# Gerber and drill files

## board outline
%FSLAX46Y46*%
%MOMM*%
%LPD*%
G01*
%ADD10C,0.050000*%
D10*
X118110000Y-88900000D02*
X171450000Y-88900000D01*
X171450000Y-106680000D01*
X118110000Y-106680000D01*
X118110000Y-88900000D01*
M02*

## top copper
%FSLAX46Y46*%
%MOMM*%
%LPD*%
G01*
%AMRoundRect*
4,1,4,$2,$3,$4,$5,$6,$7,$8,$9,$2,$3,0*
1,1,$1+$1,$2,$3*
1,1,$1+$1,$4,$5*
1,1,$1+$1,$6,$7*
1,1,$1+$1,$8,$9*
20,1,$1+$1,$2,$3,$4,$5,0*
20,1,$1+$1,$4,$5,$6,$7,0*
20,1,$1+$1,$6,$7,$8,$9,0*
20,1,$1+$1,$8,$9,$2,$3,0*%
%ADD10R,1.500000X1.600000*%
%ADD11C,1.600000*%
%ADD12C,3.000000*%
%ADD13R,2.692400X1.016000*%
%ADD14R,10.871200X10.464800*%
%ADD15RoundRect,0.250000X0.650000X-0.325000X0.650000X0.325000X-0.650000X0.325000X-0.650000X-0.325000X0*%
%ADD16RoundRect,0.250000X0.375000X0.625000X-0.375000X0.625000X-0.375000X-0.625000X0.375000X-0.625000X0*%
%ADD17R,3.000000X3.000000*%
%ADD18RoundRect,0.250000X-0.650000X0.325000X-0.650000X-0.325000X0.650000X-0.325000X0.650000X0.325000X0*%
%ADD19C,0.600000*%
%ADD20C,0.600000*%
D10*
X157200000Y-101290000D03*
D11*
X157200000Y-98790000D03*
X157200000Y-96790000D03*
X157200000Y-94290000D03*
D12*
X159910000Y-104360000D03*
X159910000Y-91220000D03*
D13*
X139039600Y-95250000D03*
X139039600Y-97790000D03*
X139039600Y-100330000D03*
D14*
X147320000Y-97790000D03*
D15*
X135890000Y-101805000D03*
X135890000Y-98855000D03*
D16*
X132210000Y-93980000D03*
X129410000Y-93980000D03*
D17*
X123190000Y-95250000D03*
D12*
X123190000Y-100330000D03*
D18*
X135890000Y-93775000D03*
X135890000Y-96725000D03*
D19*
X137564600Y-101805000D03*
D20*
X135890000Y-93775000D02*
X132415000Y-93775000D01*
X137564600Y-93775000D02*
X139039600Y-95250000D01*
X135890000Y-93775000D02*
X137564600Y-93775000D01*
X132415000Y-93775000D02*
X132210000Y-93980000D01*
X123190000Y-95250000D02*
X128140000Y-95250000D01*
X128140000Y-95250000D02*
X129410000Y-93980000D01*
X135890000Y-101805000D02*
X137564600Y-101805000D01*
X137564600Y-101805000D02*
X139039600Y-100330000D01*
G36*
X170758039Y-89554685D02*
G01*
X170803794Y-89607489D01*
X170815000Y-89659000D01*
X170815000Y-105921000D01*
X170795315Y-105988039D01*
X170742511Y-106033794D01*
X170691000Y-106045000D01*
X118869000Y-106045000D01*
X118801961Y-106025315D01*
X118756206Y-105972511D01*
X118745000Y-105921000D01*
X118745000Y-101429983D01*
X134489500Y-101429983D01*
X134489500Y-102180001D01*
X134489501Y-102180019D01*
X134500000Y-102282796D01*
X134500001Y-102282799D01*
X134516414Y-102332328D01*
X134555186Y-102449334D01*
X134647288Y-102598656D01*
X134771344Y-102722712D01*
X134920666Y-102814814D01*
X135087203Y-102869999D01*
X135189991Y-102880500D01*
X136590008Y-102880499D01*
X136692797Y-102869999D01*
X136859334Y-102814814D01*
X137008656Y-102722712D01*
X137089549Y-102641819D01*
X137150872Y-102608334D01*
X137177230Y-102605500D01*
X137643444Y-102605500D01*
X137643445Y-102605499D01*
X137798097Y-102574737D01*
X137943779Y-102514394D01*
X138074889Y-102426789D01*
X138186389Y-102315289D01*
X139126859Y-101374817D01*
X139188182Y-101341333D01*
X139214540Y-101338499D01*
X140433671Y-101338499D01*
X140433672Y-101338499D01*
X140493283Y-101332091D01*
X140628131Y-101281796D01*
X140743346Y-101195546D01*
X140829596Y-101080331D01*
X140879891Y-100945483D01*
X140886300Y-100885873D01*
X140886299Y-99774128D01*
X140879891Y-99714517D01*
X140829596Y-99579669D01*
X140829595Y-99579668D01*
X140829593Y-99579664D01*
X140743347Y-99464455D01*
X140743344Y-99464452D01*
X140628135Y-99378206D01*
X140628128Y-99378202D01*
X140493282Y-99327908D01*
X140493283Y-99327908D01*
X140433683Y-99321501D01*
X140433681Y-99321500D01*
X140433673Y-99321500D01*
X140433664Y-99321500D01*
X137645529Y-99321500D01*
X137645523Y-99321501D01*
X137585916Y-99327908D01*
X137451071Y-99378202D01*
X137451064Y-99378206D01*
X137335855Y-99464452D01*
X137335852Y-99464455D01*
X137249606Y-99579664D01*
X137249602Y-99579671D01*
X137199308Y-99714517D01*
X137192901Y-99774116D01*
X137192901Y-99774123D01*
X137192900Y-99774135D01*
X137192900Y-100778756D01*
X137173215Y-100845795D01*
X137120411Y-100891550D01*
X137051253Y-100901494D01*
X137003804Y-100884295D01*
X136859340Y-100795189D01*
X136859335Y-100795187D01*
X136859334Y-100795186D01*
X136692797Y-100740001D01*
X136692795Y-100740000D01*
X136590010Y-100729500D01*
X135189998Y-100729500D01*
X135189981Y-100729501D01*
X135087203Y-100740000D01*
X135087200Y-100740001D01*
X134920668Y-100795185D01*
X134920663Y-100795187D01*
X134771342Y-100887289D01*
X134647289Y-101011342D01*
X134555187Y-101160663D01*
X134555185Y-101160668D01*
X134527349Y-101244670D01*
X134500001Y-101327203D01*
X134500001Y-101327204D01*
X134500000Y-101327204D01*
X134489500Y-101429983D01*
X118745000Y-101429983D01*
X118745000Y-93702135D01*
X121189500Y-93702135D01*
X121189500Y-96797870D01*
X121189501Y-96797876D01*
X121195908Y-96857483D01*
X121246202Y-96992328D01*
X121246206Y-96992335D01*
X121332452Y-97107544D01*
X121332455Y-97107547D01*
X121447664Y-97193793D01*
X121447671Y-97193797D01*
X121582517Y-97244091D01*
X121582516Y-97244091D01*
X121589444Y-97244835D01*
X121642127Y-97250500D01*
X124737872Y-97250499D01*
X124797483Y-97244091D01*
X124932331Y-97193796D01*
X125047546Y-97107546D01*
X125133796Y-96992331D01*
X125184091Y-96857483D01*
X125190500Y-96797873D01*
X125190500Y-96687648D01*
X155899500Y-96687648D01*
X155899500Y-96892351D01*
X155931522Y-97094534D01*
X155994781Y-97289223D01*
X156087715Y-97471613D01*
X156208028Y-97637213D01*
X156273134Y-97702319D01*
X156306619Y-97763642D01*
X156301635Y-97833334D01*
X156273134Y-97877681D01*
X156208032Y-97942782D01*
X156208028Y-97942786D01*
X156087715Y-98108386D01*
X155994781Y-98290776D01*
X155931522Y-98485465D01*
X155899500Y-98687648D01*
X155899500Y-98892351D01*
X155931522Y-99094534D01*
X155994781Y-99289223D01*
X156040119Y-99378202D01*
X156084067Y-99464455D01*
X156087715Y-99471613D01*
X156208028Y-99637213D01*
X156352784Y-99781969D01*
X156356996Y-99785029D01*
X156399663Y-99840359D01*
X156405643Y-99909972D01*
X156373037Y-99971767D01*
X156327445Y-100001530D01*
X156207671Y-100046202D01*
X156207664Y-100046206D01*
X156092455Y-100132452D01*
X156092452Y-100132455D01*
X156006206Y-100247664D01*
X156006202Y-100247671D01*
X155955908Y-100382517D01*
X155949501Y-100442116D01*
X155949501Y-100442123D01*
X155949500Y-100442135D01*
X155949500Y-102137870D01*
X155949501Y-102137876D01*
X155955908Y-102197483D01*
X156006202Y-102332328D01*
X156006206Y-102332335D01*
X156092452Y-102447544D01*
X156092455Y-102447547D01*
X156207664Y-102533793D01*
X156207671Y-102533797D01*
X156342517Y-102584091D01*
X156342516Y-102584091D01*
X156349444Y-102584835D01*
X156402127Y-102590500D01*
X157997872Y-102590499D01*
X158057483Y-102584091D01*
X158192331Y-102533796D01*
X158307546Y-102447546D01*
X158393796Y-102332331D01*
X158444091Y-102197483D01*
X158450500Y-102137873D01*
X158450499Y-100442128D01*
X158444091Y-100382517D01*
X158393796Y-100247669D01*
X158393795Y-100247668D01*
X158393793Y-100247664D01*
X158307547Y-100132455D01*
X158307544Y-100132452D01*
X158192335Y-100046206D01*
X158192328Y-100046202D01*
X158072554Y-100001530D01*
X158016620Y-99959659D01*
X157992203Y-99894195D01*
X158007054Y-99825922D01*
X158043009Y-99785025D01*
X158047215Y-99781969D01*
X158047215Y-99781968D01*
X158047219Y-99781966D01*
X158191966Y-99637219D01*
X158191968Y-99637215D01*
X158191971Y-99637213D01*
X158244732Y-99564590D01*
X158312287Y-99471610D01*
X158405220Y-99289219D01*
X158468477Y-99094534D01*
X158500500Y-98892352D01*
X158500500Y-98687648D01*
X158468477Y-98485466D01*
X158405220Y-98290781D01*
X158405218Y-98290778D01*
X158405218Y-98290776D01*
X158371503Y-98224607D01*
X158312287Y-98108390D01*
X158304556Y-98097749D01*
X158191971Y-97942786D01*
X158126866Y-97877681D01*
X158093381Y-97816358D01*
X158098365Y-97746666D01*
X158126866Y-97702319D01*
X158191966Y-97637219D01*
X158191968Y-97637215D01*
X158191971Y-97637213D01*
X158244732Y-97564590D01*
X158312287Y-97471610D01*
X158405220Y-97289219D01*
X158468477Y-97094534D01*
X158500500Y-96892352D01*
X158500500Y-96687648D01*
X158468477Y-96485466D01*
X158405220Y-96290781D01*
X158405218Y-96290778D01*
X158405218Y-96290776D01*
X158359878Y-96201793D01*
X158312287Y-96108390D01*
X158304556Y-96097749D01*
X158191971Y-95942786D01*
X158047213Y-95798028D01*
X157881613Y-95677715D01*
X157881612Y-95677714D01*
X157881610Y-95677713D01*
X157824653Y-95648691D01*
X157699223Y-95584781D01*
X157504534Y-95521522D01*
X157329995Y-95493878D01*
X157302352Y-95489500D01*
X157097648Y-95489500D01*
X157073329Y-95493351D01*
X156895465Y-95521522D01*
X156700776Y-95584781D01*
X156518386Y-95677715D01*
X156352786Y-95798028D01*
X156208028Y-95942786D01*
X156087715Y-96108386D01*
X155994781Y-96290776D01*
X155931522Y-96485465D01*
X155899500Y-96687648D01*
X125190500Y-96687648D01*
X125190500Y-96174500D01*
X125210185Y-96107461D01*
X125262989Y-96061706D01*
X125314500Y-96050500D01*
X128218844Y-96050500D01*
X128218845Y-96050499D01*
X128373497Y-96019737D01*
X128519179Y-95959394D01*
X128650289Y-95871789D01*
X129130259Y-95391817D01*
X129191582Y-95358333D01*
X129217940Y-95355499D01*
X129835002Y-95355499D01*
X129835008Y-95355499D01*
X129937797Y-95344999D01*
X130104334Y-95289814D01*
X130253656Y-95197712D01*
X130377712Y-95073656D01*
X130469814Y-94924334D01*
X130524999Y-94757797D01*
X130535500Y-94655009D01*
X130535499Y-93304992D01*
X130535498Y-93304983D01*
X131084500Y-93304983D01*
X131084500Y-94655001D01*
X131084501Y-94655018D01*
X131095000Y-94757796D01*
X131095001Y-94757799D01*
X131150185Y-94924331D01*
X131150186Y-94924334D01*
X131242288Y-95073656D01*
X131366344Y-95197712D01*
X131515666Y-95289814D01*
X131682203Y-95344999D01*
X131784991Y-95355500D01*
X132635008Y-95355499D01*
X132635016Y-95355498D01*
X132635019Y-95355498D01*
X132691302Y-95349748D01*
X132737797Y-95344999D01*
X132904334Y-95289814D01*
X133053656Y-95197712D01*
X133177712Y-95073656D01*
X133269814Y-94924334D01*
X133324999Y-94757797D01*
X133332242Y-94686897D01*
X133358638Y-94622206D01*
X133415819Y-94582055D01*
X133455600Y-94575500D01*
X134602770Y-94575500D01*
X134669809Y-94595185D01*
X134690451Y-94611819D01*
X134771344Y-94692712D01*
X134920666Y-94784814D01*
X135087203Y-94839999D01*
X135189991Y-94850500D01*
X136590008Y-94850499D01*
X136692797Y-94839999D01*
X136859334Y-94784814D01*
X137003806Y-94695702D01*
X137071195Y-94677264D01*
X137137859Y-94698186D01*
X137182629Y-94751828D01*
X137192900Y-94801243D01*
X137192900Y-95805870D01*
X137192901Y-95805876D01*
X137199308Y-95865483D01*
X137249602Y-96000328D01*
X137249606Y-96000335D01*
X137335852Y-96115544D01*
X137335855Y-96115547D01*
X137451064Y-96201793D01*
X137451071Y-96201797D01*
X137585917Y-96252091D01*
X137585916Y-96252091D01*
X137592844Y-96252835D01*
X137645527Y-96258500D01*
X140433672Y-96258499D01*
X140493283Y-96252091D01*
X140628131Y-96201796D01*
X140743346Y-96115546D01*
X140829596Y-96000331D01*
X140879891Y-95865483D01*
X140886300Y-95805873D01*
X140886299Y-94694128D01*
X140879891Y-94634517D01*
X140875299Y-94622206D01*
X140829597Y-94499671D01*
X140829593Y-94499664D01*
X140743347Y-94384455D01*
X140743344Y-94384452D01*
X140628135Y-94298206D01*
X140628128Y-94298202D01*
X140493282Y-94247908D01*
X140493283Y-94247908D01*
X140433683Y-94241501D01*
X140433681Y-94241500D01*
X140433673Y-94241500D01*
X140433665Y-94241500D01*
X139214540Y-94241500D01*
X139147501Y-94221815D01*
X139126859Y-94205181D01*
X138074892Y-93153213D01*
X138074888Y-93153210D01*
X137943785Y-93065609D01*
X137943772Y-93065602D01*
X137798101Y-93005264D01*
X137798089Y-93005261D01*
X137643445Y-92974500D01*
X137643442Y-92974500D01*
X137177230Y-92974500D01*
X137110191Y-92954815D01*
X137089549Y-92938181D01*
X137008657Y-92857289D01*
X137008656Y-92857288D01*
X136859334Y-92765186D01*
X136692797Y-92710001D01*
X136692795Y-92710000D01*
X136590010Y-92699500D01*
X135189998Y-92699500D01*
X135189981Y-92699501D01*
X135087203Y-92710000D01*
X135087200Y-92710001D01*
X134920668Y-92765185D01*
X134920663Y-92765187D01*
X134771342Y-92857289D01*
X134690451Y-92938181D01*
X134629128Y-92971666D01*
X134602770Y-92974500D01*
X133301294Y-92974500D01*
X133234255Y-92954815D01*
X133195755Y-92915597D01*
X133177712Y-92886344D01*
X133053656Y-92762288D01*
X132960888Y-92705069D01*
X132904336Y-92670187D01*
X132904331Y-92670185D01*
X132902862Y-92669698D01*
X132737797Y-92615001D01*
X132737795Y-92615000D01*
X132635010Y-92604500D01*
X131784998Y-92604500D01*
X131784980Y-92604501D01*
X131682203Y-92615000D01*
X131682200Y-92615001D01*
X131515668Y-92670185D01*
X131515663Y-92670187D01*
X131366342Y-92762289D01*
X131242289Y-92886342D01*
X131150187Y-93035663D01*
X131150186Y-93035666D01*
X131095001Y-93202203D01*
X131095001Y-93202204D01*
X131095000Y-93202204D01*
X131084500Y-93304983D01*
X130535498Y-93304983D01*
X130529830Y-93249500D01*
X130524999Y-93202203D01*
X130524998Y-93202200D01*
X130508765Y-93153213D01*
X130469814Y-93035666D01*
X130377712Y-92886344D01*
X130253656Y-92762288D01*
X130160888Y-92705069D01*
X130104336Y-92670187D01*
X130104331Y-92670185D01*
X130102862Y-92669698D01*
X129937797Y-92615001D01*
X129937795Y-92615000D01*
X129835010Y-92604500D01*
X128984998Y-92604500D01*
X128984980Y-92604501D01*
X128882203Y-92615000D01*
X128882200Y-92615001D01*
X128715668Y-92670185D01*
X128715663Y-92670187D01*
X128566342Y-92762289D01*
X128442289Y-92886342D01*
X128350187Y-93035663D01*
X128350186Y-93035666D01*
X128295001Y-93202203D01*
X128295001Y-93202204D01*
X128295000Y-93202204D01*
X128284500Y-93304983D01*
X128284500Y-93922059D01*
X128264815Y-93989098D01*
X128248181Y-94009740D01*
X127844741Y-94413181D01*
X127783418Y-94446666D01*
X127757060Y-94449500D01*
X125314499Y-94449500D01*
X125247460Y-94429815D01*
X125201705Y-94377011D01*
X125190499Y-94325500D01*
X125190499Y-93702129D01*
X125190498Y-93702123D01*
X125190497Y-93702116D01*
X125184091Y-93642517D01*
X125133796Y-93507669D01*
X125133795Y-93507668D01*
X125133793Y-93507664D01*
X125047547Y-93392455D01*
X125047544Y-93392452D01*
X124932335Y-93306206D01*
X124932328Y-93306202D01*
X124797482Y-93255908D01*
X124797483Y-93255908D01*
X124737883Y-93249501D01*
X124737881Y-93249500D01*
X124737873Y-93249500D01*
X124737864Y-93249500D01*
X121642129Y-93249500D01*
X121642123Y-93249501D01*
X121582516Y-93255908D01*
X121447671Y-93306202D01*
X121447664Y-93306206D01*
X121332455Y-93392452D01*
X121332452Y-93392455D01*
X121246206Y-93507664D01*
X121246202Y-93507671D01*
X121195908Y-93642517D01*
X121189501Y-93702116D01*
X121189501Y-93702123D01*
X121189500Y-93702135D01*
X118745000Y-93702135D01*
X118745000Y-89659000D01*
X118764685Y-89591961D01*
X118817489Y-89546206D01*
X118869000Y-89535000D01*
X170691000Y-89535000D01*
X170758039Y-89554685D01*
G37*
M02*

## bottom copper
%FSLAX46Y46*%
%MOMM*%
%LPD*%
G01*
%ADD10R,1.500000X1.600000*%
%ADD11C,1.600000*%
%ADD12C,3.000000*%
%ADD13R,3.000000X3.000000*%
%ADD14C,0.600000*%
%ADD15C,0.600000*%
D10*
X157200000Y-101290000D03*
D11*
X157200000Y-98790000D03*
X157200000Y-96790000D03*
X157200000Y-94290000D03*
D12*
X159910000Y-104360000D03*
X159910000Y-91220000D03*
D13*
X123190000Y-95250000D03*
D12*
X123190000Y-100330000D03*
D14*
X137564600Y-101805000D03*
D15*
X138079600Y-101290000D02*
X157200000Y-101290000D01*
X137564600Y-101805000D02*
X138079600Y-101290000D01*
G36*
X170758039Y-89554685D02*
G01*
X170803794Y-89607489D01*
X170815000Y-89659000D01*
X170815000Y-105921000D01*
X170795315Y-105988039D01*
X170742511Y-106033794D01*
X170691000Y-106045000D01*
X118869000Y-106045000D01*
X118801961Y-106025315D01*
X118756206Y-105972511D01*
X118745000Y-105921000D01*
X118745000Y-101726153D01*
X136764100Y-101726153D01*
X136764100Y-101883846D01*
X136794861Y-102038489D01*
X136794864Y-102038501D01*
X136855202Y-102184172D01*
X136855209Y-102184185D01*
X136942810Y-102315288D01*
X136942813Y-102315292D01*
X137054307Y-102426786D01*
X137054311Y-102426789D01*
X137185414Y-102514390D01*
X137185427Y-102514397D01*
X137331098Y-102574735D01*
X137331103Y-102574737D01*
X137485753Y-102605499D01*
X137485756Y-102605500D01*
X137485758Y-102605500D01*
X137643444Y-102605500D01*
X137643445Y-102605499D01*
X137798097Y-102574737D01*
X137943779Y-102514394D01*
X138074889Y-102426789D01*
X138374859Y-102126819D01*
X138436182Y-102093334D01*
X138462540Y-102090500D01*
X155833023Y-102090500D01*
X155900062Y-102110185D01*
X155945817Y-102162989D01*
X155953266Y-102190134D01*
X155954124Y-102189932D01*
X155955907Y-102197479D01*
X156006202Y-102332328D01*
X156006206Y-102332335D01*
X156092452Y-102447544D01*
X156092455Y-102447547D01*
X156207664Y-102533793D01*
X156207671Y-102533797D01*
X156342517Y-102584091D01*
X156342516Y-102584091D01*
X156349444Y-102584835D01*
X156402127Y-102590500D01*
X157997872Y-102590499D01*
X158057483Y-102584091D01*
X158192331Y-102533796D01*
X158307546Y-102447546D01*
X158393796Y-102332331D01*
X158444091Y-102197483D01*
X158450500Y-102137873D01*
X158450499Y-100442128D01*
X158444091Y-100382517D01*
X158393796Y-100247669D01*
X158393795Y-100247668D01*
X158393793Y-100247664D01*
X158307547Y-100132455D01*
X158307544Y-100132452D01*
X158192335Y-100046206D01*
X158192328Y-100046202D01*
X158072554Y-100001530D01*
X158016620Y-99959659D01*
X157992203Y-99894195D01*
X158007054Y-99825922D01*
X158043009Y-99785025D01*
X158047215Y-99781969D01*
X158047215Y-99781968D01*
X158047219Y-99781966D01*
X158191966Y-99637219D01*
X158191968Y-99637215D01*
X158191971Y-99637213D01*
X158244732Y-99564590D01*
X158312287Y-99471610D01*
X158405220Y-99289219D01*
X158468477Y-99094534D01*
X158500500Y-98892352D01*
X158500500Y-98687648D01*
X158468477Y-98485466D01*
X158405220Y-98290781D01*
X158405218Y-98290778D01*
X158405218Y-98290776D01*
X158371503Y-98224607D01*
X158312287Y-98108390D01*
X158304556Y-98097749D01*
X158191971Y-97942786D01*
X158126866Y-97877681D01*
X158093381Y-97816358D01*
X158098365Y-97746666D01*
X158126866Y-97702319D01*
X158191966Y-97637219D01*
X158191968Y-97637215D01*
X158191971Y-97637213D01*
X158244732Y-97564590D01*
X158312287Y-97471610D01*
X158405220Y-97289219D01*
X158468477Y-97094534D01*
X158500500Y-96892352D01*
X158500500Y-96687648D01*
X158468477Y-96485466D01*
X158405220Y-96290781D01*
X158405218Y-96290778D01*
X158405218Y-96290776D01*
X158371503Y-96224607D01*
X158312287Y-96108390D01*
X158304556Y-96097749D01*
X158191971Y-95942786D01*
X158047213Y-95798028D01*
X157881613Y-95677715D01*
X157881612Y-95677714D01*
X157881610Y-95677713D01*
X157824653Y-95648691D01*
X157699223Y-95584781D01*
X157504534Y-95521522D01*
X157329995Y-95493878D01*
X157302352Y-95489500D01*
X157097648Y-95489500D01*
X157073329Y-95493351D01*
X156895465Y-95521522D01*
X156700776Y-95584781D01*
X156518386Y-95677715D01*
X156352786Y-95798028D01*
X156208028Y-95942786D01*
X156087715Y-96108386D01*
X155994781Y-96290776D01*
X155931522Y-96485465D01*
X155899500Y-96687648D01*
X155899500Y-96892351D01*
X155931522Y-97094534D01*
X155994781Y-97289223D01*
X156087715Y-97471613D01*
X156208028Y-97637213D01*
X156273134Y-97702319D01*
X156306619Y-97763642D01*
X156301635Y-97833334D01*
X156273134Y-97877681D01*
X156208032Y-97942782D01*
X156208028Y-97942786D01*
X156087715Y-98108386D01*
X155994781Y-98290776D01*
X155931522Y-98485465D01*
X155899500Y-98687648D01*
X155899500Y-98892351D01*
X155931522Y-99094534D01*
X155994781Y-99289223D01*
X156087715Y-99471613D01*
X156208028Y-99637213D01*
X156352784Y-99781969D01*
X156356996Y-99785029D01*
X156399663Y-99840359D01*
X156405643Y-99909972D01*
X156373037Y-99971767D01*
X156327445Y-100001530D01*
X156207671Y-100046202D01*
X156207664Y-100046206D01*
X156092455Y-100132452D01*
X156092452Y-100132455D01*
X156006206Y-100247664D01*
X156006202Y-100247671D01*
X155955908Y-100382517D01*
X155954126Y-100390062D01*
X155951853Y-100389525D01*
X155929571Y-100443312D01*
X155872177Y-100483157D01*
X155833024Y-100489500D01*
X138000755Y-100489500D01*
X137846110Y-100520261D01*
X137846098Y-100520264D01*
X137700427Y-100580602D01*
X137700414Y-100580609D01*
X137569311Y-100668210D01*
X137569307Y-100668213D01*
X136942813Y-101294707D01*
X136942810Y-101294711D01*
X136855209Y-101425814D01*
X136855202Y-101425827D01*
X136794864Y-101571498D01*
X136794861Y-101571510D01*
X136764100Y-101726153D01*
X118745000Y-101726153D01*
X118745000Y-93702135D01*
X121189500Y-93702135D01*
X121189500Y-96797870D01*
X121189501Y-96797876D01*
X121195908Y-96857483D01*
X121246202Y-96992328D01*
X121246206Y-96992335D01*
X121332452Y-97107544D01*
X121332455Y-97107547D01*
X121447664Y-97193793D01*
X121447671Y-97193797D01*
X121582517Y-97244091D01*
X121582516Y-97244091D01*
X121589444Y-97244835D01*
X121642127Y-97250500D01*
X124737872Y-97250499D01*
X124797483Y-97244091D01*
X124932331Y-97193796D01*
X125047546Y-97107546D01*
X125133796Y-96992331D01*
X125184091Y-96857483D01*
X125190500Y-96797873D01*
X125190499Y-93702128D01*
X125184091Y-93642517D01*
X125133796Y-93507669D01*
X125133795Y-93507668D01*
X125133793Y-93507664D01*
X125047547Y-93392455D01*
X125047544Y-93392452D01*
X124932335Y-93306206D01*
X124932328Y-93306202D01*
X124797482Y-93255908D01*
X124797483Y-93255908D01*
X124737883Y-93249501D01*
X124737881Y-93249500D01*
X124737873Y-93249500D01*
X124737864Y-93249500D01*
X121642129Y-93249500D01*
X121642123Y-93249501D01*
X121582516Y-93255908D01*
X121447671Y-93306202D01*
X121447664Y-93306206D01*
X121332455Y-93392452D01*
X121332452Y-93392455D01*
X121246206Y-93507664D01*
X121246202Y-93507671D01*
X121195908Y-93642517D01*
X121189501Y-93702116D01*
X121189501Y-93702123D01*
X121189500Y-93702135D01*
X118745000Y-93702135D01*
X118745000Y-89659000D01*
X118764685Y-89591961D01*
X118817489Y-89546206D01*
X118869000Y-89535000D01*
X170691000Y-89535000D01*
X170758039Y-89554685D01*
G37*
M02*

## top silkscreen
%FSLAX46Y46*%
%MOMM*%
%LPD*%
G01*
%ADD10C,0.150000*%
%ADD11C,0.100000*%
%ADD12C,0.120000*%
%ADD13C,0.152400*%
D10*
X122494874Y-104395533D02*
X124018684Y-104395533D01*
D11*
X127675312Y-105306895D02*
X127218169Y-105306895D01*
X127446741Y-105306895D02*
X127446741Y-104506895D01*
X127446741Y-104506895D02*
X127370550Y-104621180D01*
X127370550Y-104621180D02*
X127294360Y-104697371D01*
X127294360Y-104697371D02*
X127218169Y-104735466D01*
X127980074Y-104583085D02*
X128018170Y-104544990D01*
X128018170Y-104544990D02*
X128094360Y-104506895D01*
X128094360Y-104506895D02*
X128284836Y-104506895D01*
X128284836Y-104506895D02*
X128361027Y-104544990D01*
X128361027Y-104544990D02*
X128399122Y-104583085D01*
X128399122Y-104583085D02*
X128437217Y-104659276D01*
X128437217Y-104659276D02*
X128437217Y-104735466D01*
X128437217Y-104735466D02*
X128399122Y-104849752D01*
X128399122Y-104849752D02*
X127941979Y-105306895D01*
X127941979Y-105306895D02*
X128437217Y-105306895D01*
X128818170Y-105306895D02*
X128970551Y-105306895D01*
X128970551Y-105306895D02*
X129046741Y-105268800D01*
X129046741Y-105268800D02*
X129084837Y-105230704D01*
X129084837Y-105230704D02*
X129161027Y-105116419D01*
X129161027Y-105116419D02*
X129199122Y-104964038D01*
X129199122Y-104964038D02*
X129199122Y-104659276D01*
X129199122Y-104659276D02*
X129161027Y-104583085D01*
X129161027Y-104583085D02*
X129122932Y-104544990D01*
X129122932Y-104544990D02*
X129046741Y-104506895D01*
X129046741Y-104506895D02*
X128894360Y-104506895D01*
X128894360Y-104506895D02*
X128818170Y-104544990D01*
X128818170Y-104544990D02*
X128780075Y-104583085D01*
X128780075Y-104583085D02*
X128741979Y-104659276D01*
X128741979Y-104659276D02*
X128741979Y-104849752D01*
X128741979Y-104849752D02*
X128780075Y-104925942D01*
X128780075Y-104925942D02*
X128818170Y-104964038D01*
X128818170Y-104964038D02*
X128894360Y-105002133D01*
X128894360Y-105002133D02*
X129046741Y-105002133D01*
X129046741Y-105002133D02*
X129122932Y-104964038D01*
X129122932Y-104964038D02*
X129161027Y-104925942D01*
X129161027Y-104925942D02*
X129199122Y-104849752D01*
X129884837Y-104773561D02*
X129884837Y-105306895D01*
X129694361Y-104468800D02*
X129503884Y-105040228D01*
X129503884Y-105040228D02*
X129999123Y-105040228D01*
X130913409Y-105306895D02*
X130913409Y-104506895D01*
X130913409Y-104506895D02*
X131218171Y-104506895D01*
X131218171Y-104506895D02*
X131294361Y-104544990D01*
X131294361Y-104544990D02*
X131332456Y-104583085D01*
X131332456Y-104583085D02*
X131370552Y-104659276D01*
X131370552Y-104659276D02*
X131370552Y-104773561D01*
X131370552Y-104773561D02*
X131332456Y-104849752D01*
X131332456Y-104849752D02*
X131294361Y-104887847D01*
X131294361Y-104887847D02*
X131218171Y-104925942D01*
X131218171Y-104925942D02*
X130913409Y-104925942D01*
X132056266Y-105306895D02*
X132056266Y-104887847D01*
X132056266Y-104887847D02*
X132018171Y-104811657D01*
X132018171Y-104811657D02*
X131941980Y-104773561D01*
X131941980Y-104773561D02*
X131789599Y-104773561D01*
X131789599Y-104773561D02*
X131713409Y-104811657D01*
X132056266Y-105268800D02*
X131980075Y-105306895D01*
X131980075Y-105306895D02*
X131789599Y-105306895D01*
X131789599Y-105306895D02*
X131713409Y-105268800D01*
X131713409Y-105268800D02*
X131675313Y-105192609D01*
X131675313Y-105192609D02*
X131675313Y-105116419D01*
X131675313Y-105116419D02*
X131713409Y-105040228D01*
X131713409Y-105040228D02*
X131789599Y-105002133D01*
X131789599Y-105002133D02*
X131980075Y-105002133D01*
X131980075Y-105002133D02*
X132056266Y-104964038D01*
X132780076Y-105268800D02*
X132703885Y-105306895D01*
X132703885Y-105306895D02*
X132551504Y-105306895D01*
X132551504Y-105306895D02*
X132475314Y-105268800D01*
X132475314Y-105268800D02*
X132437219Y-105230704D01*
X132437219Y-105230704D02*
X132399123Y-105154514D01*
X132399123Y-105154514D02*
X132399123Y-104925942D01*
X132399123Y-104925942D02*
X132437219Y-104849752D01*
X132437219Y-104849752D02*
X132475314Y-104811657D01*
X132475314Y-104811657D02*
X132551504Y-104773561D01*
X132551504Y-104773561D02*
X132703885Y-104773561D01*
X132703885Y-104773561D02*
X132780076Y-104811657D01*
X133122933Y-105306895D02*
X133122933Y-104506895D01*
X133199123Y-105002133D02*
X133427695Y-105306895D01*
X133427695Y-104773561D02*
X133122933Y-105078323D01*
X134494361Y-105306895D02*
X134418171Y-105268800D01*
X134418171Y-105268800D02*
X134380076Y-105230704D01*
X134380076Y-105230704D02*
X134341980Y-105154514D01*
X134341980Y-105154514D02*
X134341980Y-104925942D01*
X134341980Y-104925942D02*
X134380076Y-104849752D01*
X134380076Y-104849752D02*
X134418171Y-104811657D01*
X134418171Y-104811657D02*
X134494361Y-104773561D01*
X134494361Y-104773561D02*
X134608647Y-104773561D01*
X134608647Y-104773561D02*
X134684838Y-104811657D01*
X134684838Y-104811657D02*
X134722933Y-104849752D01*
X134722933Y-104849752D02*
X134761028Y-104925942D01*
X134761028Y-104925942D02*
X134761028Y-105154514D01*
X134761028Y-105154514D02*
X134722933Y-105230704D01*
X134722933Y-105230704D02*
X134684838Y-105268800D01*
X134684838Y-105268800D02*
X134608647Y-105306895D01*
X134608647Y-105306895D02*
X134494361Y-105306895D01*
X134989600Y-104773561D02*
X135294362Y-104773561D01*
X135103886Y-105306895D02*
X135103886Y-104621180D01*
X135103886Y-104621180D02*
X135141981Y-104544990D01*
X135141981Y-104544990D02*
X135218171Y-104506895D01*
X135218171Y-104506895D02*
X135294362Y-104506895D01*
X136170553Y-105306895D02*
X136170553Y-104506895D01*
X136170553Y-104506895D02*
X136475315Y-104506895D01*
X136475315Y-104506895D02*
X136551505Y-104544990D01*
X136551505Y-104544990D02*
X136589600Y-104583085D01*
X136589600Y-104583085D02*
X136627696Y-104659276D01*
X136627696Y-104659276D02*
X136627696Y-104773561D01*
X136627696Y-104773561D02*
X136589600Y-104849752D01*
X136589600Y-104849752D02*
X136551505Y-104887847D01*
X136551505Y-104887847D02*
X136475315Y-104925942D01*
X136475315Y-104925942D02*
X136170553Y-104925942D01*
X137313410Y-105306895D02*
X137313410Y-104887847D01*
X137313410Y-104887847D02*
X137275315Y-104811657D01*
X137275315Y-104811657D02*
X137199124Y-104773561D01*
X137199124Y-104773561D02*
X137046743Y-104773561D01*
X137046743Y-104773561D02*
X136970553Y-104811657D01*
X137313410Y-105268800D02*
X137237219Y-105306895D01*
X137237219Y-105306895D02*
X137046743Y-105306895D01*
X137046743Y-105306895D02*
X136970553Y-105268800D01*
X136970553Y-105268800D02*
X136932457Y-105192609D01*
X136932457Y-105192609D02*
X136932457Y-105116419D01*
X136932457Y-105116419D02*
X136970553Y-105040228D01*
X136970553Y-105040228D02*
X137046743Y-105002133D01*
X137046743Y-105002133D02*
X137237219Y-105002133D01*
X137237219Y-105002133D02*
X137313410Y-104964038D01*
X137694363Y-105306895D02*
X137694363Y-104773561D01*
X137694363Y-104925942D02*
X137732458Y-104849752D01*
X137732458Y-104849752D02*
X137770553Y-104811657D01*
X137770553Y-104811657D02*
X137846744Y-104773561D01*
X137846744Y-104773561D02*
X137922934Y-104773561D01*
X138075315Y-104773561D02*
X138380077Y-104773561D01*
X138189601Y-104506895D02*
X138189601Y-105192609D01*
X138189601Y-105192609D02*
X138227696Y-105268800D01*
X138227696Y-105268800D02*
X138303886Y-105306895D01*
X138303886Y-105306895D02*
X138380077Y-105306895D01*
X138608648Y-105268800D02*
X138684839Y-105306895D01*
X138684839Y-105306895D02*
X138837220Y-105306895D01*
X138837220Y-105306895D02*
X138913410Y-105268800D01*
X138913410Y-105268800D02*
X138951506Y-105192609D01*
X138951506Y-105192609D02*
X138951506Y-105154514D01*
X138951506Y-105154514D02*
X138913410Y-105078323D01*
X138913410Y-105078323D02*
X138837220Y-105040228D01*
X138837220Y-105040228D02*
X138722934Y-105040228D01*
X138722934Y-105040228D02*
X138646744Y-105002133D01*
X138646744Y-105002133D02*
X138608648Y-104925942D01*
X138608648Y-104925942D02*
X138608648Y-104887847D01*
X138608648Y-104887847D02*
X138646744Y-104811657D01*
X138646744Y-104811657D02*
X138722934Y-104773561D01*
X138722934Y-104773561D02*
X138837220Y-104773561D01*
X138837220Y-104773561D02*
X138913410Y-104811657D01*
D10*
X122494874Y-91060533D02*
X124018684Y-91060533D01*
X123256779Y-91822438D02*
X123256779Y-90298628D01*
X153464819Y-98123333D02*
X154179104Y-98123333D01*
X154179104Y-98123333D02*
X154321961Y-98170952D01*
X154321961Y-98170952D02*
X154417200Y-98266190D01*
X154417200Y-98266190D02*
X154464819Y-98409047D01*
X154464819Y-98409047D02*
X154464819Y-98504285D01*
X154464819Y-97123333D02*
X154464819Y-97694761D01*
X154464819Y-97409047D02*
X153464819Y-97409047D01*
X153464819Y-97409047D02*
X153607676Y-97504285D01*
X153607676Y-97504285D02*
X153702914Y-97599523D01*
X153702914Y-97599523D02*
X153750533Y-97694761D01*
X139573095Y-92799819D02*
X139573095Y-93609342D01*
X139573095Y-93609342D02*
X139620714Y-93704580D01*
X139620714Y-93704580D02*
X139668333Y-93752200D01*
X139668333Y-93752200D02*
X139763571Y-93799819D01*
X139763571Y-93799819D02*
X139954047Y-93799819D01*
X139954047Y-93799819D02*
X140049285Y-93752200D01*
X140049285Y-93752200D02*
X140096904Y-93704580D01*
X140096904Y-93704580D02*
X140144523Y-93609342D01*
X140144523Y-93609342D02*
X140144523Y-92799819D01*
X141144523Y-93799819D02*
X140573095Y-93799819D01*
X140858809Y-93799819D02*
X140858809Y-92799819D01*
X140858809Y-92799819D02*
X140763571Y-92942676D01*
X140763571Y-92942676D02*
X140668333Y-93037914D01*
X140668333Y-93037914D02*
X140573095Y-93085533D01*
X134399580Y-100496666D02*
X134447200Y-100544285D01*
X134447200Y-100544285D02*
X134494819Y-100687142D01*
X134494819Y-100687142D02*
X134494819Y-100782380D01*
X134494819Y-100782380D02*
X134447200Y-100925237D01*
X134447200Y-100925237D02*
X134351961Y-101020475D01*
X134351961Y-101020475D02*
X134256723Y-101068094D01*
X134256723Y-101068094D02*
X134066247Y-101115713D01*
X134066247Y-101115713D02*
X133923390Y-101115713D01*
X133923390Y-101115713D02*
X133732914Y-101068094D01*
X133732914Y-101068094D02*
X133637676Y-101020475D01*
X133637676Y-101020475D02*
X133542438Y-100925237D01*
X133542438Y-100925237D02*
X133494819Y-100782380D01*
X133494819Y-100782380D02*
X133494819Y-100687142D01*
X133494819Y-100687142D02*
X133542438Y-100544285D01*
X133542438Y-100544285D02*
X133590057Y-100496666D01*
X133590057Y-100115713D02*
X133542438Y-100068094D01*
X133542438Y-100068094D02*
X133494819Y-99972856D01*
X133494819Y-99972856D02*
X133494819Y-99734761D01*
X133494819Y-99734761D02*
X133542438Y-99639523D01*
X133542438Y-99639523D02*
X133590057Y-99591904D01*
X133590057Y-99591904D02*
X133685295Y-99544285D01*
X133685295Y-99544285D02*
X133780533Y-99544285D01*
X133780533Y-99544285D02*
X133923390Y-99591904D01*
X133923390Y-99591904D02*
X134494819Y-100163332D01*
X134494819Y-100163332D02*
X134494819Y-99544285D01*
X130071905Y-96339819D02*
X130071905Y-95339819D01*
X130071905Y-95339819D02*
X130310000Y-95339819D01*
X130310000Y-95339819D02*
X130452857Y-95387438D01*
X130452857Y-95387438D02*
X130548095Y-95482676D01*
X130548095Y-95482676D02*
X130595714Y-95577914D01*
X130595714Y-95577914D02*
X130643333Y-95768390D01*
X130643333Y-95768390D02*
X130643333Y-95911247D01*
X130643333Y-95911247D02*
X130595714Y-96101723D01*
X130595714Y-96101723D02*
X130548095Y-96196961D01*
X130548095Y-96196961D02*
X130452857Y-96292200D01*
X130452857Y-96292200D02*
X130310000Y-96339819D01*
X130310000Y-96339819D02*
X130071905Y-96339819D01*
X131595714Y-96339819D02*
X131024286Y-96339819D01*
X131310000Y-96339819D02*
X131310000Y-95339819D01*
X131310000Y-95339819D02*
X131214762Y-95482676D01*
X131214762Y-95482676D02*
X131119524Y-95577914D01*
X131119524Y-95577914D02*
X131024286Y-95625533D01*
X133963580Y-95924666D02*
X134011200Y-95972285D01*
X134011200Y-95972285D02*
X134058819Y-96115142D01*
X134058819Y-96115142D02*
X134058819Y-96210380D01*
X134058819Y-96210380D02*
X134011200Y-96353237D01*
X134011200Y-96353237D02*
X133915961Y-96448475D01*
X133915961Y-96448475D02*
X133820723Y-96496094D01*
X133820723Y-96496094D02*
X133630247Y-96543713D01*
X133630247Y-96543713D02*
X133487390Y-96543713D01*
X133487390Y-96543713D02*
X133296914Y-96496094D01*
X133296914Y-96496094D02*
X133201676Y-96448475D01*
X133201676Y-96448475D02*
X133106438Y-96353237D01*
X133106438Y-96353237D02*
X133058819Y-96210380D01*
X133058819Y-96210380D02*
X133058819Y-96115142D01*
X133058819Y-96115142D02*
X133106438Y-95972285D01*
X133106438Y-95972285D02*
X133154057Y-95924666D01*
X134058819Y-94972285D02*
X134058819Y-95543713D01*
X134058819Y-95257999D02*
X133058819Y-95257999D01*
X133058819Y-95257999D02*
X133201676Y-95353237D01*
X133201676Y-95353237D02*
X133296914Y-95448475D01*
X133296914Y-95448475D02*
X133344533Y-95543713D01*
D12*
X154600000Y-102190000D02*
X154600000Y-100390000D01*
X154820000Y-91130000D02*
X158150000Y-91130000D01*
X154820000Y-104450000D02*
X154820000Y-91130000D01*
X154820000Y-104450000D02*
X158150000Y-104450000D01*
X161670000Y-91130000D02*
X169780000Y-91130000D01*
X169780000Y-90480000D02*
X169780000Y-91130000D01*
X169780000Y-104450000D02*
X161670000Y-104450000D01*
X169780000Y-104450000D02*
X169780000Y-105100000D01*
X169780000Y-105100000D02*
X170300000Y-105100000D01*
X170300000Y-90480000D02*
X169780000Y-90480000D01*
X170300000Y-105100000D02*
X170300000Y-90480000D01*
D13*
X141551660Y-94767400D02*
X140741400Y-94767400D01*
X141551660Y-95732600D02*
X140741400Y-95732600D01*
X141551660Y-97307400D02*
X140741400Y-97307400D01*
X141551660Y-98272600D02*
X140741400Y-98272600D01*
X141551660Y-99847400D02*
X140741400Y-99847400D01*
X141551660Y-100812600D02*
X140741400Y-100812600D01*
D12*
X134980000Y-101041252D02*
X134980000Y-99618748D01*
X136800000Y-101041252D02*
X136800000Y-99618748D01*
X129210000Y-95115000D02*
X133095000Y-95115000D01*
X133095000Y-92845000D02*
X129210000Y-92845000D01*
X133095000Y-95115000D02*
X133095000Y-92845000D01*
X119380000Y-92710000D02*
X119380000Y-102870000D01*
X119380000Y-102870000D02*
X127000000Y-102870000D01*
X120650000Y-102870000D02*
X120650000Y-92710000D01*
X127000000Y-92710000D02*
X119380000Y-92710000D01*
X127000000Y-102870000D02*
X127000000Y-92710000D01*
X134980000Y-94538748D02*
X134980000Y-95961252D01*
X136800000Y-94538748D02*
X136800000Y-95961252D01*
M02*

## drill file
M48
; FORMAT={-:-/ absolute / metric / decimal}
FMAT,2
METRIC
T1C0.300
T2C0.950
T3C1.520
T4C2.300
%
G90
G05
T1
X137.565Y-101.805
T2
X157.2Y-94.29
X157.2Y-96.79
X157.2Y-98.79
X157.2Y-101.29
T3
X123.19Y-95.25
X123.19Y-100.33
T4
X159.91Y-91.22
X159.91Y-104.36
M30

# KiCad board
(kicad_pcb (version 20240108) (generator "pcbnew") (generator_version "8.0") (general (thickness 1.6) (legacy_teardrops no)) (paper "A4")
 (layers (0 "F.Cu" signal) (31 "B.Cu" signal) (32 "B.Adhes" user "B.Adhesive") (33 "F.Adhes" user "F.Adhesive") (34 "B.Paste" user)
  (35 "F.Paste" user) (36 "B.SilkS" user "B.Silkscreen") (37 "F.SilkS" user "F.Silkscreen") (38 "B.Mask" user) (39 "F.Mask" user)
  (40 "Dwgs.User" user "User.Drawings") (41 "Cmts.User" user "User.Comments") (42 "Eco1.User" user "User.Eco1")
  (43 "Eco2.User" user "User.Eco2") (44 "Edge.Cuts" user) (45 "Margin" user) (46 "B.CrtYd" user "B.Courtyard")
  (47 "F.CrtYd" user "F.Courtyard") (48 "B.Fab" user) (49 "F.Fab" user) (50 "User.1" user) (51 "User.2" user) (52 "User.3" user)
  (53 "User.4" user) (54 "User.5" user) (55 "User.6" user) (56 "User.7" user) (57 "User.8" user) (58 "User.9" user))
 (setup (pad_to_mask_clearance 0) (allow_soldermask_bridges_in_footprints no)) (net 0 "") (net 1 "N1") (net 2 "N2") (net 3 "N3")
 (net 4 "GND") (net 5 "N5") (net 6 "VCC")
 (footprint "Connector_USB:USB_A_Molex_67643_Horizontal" (layer "F.Cu") (at 157.2 101.29 90)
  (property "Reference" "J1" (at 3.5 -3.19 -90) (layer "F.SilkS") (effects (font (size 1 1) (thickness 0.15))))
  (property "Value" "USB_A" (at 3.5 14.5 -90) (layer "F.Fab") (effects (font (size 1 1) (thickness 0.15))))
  (fp_line (start -0.9 -2.6) (end 0.9 -2.6) (stroke (width 0.12) (type solid)) (layer "F.SilkS"))
  (fp_line (start 10.16 -2.38) (end 10.16 0.95) (stroke (width 0.12) (type solid)) (layer "F.SilkS"))
  (fp_line (start -3.16 -2.38) (end 10.16 -2.38) (stroke (width 0.12) (type solid)) (layer "F.SilkS"))
  (fp_line (start -3.16 -2.38) (end -3.16 0.95) (stroke (width 0.12) (type solid)) (layer "F.SilkS"))
  (fp_line (start 10.16 4.47) (end 10.16 12.58) (stroke (width 0.12) (type solid)) (layer "F.SilkS"))
  (fp_line (start 10.81 12.58) (end 10.16 12.58) (stroke (width 0.12) (type solid)) (layer "F.SilkS"))
  (fp_line (start -3.16 12.58) (end -3.16 4.47) (stroke (width 0.12) (type solid)) (layer "F.SilkS"))
  (fp_line (start -3.16 12.58) (end -3.81 12.58) (stroke (width 0.12) (type solid)) (layer "F.SilkS"))
  (fp_line (start -3.81 12.58) (end -3.81 13.1) (stroke (width 0.12) (type solid)) (layer "F.SilkS"))
  (fp_line (start 10.81 13.1) (end 10.81 12.58) (stroke (width 0.12) (type solid)) (layer "F.SilkS"))
  (fp_line (start -3.81 13.1) (end 10.81 13.1) (stroke (width 0.12) (type solid)) (layer "F.SilkS"))
  (pad "1" thru_hole rect (at 0 0 90) (size 1.6 1.5) (drill 0.95) (layers "*.Cu" "*.Mask") (remove_unused_layers no) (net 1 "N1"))
  (pad "2" thru_hole circle (at 2.5 0 90) (size 1.6 1.6) (drill 0.95) (layers "*.Cu" "*.Mask") (remove_unused_layers no) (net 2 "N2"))
  (pad "3" thru_hole circle (at 4.5 0 90) (size 1.6 1.6) (drill 0.95) (layers "*.Cu" "*.Mask") (remove_unused_layers no) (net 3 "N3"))
  (pad "4" thru_hole circle (at 7 0 90) (size 1.6 1.6) (drill 0.95) (layers "*.Cu" "*.Mask") (remove_unused_layers no) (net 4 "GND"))
  (pad "5" thru_hole circle (at -3.07 2.71 90) (size 3 3) (drill 2.3) (layers "*.Cu" "*.Mask") (remove_unused_layers no) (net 4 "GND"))
  (pad "5" thru_hole circle (at 10.07 2.71 90) (size 3 3) (drill 2.3) (layers "*.Cu" "*.Mask") (remove_unused_layers no) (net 4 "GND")))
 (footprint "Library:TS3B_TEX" (layer "F.Cu") (at 147.32 97.79 -90)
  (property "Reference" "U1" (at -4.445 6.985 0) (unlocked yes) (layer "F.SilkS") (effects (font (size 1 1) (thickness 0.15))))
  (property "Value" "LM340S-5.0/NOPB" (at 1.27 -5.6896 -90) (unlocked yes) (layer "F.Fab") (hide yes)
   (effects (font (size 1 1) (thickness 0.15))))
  (fp_line (start -3.0226 5.76834) (end -3.0226 6.5786) (stroke (width 0.1524) (type solid)) (layer "F.SilkS"))
  (fp_line (start -2.0574 5.76834) (end -2.0574 6.5786) (stroke (width 0.1524) (type solid)) (layer "F.SilkS"))
  (fp_line (start -0.4826 5.76834) (end -0.4826 6.5786) (stroke (width 0.1524) (type solid)) (layer "F.SilkS"))
  (fp_line (start 0.4826 5.76834) (end 0.4826 6.5786) (stroke (width 0.1524) (type solid)) (layer "F.SilkS"))
  (fp_line (start 2.0574 5.76834) (end 2.0574 6.5786) (stroke (width 0.1524) (type solid)) (layer "F.SilkS"))
  (fp_line (start 3.0226 5.76834) (end 3.0226 6.5786) (stroke (width 0.1524) (type solid)) (layer "F.SilkS"))
  (pad "1" smd rect (at -2.54 8.2804 270) (size 1.016 2.6924) (layers "F.Cu" "F.Paste" "F.Mask") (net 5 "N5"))
  (pad "2" smd rect (at 0 8.2804 270) (size 1.016 2.6924) (layers "F.Cu" "F.Paste" "F.Mask") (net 4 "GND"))
  (pad "3" smd rect (at 2.54 8.2804 270) (size 1.016 2.6924) (layers "F.Cu" "F.Paste" "F.Mask") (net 1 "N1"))
  (pad "4" smd rect (at 0 0 270) (size 10.4648 10.8712) (layers "F.Cu" "F.Paste" "F.Mask") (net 4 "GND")))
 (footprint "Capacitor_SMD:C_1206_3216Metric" (layer "F.Cu") (at 135.89 100.33 90)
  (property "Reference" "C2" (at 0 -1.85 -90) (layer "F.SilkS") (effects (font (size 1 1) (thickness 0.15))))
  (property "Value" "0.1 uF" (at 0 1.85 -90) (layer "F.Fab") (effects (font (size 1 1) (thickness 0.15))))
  (fp_line (start -0.711252 -0.91) (end 0.711252 -0.91) (stroke (width 0.12) (type solid)) (layer "F.SilkS"))
  (fp_line (start -0.711252 0.91) (end 0.711252 0.91) (stroke (width 0.12) (type solid)) (layer "F.SilkS"))
  (pad "1" smd roundrect (at -1.475 0 90) (size 1.15 1.8) (layers "F.Cu" "F.Paste" "F.Mask") (roundrect_rratio 0.217391) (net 1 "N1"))
  (pad "2" smd roundrect (at 1.475 0 90) (size 1.15 1.8) (layers "F.Cu" "F.Paste" "F.Mask") (roundrect_rratio 0.217391) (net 4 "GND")))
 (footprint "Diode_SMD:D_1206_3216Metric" (layer "F.Cu") (at 130.81 93.98 180)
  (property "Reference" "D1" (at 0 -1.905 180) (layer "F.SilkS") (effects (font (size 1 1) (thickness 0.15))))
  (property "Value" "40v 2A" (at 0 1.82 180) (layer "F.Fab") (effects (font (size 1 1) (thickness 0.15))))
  (fp_line (start 1.6 -1.135) (end -2.285 -1.135) (stroke (width 0.12) (type solid)) (layer "F.SilkS"))
  (fp_line (start -2.285 1.135) (end 1.6 1.135) (stroke (width 0.12) (type solid)) (layer "F.SilkS"))
  (fp_line (start -2.285 -1.135) (end -2.285 1.135) (stroke (width 0.12) (type solid)) (layer "F.SilkS"))
  (pad "1" smd roundrect (at -1.4 0 180) (size 1.25 1.75) (layers "F.Cu" "F.Paste" "F.Mask") (roundrect_rratio 0.2) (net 5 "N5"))
  (pad "2" smd roundrect (at 1.4 0 180) (size 1.25 1.75) (layers "F.Cu" "F.Paste" "F.Mask") (roundrect_rratio 0.2) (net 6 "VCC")))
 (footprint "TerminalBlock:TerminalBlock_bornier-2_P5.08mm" (layer "F.Cu") (at 123.19 95.25 -90)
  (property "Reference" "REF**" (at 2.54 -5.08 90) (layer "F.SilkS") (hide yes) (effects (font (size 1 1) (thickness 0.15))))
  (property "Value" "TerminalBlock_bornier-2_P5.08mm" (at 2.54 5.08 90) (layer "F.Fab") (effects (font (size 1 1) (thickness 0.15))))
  (fp_line (start -2.54 3.81) (end 7.62 3.81) (stroke (width 0.12) (type solid)) (layer "F.SilkS"))
  (fp_line (start 7.62 3.81) (end 7.62 -3.81) (stroke (width 0.12) (type solid)) (layer "F.SilkS"))
  (fp_line (start 7.62 2.54) (end -2.54 2.54) (stroke (width 0.12) (type solid)) (layer "F.SilkS"))
  (fp_line (start -2.54 -3.81) (end -2.54 3.81) (stroke (width 0.12) (type solid)) (layer "F.SilkS"))
  (fp_line (start 7.62 -3.81) (end -2.54 -3.81) (stroke (width 0.12) (type solid)) (layer "F.SilkS"))
  (pad "1" thru_hole rect (at 0 0 270) (size 3 3) (drill 1.52) (layers "*.Cu" "*.Mask") (remove_unused_layers no) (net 6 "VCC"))
  (pad "2" thru_hole circle (at 5.08 0 270) (size 3 3) (drill 1.52) (layers "*.Cu" "*.Mask") (remove_unused_layers no) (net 4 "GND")))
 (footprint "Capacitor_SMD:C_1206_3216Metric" (layer "F.Cu") (at 135.89 95.25 -90)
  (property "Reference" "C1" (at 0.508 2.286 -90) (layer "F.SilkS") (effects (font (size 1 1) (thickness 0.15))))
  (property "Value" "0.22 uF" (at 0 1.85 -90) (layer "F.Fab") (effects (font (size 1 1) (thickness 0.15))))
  (fp_line (start -0.711252 0.91) (end 0.711252 0.91) (stroke (width 0.12) (type solid)) (layer "F.SilkS"))
  (fp_line (start -0.711252 -0.91) (end 0.711252 -0.91) (stroke (width 0.12) (type solid)) (layer "F.SilkS"))
  (pad "1" smd roundrect (at -1.475 0 270) (size 1.15 1.8) (layers "F.Cu" "F.Paste" "F.Mask") (roundrect_rratio 0.217391) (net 5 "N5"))
  (pad "2" smd roundrect (at 1.475 0 270) (size 1.15 1.8) (layers "F.Cu" "F.Paste" "F.Mask") (roundrect_rratio 0.217391) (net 4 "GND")))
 (gr_rect (start 118.11 88.9) (end 171.45 106.68) (stroke (width 0.05) (type default)) (fill none) (layer "Edge.Cuts"))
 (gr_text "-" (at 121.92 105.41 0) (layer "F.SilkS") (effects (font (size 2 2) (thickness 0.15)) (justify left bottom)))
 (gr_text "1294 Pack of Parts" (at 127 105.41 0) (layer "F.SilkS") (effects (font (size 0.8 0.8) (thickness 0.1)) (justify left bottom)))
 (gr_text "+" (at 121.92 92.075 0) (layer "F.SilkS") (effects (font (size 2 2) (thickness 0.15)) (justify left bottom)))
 (segment (start 135.89 93.775) (end 132.415 93.775) (width 0.6) (layer "F.Cu") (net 5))
 (segment (start 137.5646 93.775) (end 139.0396 95.25) (width 0.6) (layer "F.Cu") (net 5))
 (segment (start 135.89 93.775) (end 137.5646 93.775) (width 0.6) (layer "F.Cu") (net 5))
 (segment (start 132.415 93.775) (end 132.21 93.98) (width 0.6) (layer "F.Cu") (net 5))
 (segment (start 123.19 95.25) (end 128.14 95.25) (width 0.6) (layer "F.Cu") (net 6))
 (segment (start 128.14 95.25) (end 129.41 93.98) (width 0.6) (layer "F.Cu") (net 6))
 (segment (start 135.89 101.805) (end 137.5646 101.805) (width 0.6) (layer "F.Cu") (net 1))
 (segment (start 137.5646 101.805) (end 139.0396 100.33) (width 0.6) (layer "F.Cu") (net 1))
 (via (at 137.5646 101.805) (size 0.6) (drill 0.3) (layers "F.Cu" "B.Cu") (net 1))
 (segment (start 138.0796 101.29) (end 157.2 101.29) (width 0.6) (layer "B.Cu") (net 1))
 (segment (start 137.5646 101.805) (end 138.0796 101.29) (width 0.6) (layer "B.Cu") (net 1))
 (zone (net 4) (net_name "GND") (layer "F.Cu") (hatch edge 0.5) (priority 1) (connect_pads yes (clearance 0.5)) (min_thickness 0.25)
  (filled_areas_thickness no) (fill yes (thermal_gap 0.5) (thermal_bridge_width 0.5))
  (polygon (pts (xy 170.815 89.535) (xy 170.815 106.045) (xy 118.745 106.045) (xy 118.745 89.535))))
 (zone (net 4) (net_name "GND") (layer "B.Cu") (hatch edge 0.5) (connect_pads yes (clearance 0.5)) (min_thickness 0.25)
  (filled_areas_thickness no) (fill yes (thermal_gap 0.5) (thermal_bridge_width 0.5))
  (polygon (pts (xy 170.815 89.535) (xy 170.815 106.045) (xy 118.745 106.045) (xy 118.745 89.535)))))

